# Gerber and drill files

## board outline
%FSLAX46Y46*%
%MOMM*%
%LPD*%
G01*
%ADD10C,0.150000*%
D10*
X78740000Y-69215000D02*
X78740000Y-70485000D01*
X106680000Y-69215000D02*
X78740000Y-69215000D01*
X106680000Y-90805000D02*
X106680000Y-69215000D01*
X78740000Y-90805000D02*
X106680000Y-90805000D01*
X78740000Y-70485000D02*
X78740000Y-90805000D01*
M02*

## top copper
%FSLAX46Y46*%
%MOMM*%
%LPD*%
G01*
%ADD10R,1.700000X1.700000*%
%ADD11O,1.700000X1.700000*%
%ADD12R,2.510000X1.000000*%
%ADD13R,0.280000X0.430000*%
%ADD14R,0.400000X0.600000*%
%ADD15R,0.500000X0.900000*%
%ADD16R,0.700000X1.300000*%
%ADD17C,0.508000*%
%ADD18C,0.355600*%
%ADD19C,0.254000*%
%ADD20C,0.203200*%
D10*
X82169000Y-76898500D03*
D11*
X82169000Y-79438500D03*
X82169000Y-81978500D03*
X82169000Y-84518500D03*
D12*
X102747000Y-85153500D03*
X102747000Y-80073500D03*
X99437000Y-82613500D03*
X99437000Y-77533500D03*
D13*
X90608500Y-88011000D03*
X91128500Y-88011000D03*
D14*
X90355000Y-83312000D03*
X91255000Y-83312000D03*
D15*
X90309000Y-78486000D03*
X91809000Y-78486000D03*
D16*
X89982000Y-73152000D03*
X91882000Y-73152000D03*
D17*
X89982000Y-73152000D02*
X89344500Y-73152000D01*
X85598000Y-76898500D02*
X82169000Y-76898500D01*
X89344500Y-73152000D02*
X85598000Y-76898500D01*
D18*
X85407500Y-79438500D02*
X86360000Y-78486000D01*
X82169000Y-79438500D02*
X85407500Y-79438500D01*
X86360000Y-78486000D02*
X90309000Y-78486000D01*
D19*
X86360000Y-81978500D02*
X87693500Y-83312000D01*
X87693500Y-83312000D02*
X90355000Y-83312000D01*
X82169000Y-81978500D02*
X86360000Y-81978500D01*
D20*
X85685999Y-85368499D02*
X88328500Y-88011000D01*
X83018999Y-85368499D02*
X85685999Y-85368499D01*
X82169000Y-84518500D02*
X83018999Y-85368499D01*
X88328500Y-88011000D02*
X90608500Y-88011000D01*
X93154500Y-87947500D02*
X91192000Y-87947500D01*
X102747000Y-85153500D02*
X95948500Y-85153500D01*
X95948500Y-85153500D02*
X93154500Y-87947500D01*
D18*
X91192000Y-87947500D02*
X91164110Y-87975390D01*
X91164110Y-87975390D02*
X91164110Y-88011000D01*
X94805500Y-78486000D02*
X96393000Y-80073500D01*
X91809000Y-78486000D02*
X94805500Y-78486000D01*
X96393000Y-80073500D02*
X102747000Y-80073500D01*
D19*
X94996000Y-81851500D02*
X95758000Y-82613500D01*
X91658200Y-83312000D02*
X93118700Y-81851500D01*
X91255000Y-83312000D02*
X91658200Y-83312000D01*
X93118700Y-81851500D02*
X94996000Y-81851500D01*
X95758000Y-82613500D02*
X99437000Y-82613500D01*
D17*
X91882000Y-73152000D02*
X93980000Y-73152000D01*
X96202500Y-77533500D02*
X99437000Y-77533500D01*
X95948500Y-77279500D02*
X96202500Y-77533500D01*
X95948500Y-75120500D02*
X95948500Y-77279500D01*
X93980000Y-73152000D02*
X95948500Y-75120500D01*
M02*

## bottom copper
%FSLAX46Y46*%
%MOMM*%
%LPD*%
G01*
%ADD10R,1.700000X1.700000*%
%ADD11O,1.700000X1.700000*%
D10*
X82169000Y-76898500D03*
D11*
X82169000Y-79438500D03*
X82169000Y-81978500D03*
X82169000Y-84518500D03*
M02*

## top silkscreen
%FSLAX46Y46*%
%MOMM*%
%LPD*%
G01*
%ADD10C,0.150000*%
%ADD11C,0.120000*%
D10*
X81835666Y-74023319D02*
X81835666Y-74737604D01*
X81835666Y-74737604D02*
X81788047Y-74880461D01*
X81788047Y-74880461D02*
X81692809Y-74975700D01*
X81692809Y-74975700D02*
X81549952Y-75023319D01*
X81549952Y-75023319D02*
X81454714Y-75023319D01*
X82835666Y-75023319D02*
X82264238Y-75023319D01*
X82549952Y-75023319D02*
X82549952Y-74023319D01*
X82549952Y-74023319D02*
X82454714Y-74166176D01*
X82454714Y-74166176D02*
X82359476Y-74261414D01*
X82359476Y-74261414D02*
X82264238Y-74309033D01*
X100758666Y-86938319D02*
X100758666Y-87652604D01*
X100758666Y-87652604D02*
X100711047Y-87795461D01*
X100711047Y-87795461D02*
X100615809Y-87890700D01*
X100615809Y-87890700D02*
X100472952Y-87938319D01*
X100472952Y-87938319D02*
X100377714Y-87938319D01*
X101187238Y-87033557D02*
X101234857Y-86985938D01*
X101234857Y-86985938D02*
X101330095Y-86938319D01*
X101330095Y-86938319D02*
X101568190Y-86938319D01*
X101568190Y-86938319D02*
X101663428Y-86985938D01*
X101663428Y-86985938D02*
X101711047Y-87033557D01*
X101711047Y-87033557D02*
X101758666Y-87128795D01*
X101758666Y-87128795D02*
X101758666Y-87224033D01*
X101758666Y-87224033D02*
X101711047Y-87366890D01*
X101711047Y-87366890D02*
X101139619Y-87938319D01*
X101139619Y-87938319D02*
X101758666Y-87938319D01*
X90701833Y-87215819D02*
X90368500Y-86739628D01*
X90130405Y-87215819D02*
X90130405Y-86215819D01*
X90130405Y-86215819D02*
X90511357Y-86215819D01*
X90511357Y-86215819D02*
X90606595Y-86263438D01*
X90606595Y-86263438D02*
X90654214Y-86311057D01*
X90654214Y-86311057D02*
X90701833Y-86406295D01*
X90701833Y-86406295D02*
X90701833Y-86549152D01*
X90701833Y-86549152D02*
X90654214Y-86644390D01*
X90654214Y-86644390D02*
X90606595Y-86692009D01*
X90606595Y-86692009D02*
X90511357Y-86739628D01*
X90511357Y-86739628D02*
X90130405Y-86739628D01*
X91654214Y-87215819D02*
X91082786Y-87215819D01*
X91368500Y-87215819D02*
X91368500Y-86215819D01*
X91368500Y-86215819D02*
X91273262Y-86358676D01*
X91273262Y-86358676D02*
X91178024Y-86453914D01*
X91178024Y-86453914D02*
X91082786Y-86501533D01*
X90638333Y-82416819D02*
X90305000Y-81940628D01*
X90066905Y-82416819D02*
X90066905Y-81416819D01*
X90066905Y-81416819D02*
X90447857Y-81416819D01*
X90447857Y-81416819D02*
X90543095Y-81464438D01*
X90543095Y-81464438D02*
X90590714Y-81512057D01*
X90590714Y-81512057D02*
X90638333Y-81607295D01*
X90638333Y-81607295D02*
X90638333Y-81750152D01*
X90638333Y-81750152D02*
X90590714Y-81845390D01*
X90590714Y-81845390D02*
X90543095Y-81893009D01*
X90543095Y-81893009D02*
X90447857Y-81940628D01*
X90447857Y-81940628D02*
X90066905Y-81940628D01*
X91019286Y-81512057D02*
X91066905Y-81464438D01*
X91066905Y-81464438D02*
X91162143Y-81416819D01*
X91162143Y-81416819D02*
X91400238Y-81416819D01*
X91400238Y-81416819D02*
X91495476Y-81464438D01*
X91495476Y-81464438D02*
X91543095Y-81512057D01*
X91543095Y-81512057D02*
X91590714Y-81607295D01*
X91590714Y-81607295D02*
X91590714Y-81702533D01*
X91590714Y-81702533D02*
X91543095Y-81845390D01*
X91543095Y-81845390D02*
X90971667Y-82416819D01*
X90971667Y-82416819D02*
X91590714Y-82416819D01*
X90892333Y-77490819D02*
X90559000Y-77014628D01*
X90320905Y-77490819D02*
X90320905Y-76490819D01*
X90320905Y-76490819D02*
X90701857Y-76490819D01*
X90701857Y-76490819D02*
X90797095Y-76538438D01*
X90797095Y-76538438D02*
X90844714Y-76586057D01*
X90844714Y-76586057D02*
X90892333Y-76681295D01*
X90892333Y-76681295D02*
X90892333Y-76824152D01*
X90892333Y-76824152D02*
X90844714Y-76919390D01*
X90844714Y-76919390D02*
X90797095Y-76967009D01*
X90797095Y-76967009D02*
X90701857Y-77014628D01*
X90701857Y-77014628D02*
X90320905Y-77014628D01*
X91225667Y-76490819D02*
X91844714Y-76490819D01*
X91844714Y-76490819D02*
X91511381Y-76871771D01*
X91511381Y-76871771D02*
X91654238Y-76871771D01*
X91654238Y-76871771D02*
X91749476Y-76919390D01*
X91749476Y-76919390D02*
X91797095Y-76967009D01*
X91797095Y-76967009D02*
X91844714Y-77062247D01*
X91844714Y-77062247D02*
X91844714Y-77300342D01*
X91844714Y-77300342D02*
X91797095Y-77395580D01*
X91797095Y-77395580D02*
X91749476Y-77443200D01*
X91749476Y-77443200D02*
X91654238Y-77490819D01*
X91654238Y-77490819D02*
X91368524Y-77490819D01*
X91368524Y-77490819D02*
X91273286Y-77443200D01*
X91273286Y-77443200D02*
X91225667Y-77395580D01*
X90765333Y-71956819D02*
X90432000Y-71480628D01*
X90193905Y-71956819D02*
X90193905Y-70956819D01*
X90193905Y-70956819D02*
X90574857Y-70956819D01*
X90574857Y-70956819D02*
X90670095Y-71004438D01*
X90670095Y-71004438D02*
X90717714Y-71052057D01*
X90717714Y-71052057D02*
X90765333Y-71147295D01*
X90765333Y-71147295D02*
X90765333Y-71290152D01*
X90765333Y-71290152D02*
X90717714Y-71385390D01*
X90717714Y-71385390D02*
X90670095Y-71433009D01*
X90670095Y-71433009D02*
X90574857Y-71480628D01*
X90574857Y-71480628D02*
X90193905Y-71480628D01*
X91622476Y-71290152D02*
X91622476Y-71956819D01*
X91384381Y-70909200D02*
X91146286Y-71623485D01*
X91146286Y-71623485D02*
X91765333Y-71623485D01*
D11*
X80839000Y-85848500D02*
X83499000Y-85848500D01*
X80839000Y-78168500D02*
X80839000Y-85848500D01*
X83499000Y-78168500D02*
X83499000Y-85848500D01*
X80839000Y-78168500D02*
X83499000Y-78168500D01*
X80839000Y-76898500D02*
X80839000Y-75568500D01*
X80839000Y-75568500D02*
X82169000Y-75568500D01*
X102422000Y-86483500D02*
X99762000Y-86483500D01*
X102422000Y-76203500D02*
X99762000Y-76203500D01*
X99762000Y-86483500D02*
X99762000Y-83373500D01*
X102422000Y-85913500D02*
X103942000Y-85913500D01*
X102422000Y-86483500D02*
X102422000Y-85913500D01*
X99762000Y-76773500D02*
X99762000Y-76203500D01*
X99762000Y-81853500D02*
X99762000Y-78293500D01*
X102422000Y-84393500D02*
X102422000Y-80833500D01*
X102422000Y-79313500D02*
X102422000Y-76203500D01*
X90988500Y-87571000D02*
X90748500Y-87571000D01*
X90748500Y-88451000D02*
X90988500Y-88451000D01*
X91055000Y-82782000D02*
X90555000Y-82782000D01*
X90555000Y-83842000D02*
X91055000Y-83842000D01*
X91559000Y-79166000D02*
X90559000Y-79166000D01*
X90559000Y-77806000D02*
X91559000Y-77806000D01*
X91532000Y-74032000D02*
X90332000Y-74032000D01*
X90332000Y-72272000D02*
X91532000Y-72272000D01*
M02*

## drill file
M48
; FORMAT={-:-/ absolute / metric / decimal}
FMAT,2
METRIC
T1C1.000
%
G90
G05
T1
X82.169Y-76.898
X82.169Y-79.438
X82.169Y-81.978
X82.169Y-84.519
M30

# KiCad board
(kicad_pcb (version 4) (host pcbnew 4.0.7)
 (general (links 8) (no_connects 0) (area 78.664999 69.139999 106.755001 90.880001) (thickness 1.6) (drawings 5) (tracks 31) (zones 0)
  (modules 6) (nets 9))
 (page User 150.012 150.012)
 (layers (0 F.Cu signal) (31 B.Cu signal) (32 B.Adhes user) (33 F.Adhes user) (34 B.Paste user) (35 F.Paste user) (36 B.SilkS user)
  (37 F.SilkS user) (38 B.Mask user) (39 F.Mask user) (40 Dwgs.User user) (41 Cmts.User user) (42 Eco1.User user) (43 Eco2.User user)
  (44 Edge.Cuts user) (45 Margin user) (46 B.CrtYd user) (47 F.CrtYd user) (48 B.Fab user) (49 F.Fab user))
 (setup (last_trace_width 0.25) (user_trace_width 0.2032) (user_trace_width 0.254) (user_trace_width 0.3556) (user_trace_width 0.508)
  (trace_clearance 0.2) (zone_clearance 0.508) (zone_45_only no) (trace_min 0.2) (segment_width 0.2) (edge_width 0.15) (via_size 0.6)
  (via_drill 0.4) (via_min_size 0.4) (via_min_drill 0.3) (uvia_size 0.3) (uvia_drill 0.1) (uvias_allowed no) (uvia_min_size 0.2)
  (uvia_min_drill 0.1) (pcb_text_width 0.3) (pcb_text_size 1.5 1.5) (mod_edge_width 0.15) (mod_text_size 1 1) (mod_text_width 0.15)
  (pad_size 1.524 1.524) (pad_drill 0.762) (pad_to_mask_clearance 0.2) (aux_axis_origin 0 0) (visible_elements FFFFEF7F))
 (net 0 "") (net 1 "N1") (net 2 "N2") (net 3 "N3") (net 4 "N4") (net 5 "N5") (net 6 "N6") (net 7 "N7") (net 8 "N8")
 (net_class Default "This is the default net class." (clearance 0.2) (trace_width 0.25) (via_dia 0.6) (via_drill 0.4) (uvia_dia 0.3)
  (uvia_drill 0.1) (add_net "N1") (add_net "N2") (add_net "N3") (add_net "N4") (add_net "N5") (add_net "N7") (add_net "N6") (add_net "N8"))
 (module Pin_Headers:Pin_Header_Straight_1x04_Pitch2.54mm (layer F.Cu) (at 82.169 76.8985)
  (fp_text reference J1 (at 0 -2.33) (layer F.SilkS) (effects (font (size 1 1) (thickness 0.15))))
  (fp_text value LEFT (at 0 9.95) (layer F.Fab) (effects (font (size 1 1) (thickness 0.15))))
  (fp_line (start -1.33 8.95) (end 1.33 8.95) (layer F.SilkS) (width 0.12))
  (fp_line (start -1.33 1.27) (end -1.33 8.95) (layer F.SilkS) (width 0.12))
  (fp_line (start 1.33 1.27) (end 1.33 8.95) (layer F.SilkS) (width 0.12))
  (fp_line (start -1.33 1.27) (end 1.33 1.27) (layer F.SilkS) (width 0.12))
  (fp_line (start -1.33 0) (end -1.33 -1.33) (layer F.SilkS) (width 0.12))
  (fp_line (start -1.33 -1.33) (end 0 -1.33) (layer F.SilkS) (width 0.12))
  (pad 1 thru_hole rect (at 0 0) (size 1.7 1.7) (drill 1) (layers *.Cu *.Mask) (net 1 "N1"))
  (pad 2 thru_hole oval (at 0 2.54) (size 1.7 1.7) (drill 1) (layers *.Cu *.Mask) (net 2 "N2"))
  (pad 3 thru_hole oval (at 0 5.08) (size 1.7 1.7) (drill 1) (layers *.Cu *.Mask) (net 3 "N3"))
  (pad 4 thru_hole oval (at 0 7.62) (size 1.7 1.7) (drill 1) (layers *.Cu *.Mask) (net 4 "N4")))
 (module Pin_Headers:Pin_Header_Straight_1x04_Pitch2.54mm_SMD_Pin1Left (layer F.Cu) (at 101.092 81.3435 180)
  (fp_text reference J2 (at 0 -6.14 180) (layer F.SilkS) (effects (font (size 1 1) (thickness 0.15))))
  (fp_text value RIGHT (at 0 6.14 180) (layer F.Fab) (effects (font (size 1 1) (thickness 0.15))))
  (fp_line (start -1.33 -5.14) (end 1.33 -5.14) (layer F.SilkS) (width 0.12))
  (fp_line (start -1.33 5.14) (end 1.33 5.14) (layer F.SilkS) (width 0.12))
  (fp_line (start 1.33 -5.14) (end 1.33 -2.03) (layer F.SilkS) (width 0.12))
  (fp_line (start -1.33 -4.57) (end -2.85 -4.57) (layer F.SilkS) (width 0.12))
  (fp_line (start -1.33 -5.14) (end -1.33 -4.57) (layer F.SilkS) (width 0.12))
  (fp_line (start 1.33 4.57) (end 1.33 5.14) (layer F.SilkS) (width 0.12))
  (fp_line (start 1.33 -0.51) (end 1.33 3.05) (layer F.SilkS) (width 0.12))
  (fp_line (start -1.33 -3.05) (end -1.33 0.51) (layer F.SilkS) (width 0.12))
  (fp_line (start -1.33 2.03) (end -1.33 5.14) (layer F.SilkS) (width 0.12))
  (pad 1 smd rect (at -1.655 -3.81 180) (size 2.51 1) (layers F.Cu F.Paste F.Mask) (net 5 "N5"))
  (pad 3 smd rect (at -1.655 1.27 180) (size 2.51 1) (layers F.Cu F.Paste F.Mask) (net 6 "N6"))
  (pad 2 smd rect (at 1.655 -1.27 180) (size 2.51 1) (layers F.Cu F.Paste F.Mask) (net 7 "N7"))
  (pad 4 smd rect (at 1.655 3.81 180) (size 2.51 1) (layers F.Cu F.Paste F.Mask) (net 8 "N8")))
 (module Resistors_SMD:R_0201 (layer F.Cu) (at 90.8685 88.011)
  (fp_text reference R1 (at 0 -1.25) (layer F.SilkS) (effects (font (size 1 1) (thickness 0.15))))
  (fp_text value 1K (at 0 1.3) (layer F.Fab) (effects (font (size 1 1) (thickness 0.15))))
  (fp_line (start 0.12 -0.44) (end -0.12 -0.44) (layer F.SilkS) (width 0.12))
  (fp_line (start -0.12 0.44) (end 0.12 0.44) (layer F.SilkS) (width 0.12))
  (pad 1 smd rect (at -0.26 0) (size 0.28 0.43) (layers F.Cu F.Paste F.Mask) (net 4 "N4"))
  (pad 2 smd rect (at 0.26 0) (size 0.28 0.43) (layers F.Cu F.Paste F.Mask) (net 5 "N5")))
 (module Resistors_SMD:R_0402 (layer F.Cu) (at 90.805 83.312)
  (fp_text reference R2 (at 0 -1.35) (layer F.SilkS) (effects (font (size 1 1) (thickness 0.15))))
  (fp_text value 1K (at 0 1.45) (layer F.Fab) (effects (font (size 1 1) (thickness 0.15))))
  (fp_line (start 0.25 -0.53) (end -0.25 -0.53) (layer F.SilkS) (width 0.12))
  (fp_line (start -0.25 0.53) (end 0.25 0.53) (layer F.SilkS) (width 0.12))
  (pad 1 smd rect (at -0.45 0) (size 0.4 0.6) (layers F.Cu F.Paste F.Mask) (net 3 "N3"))
  (pad 2 smd rect (at 0.45 0) (size 0.4 0.6) (layers F.Cu F.Paste F.Mask) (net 7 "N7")))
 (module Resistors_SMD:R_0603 (layer F.Cu) (at 91.059 78.486)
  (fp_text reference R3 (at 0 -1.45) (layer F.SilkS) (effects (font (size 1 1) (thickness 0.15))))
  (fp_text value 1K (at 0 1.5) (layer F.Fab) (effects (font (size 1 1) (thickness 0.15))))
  (fp_line (start 0.5 0.68) (end -0.5 0.68) (layer F.SilkS) (width 0.12))
  (fp_line (start -0.5 -0.68) (end 0.5 -0.68) (layer F.SilkS) (width 0.12))
  (pad 1 smd rect (at -0.75 0) (size 0.5 0.9) (layers F.Cu F.Paste F.Mask) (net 2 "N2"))
  (pad 2 smd rect (at 0.75 0) (size 0.5 0.9) (layers F.Cu F.Paste F.Mask) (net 6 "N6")))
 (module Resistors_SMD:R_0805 (layer F.Cu) (at 90.932 73.152)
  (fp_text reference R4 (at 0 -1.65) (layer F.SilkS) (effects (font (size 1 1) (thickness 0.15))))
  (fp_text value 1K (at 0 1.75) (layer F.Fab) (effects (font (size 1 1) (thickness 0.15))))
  (fp_line (start 0.6 0.88) (end -0.6 0.88) (layer F.SilkS) (width 0.12))
  (fp_line (start -0.6 -0.88) (end 0.6 -0.88) (layer F.SilkS) (width 0.12))
  (pad 1 smd rect (at -0.95 0) (size 0.7 1.3) (layers F.Cu F.Paste F.Mask) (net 1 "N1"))
  (pad 2 smd rect (at 0.95 0) (size 0.7 1.3) (layers F.Cu F.Paste F.Mask) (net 8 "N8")))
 (gr_line (start 78.74 69.215) (end 78.74 70.485) (layer Edge.Cuts) (width 0.15))
 (gr_line (start 106.68 69.215) (end 78.74 69.215) (layer Edge.Cuts) (width 0.15))
 (gr_line (start 106.68 90.805) (end 106.68 69.215) (layer Edge.Cuts) (width 0.15))
 (gr_line (start 78.74 90.805) (end 106.68 90.805) (layer Edge.Cuts) (width 0.15))
 (gr_line (start 78.74 70.485) (end 78.74 90.805) (layer Edge.Cuts) (width 0.15))
 (segment (start 89.982 73.152) (end 89.3445 73.152) (width 0.508) (layer F.Cu) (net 1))
 (segment (start 85.598 76.8985) (end 82.169 76.8985) (width 0.508) (layer F.Cu) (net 1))
 (segment (start 89.3445 73.152) (end 85.598 76.8985) (width 0.508) (layer F.Cu) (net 1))
 (segment (start 85.4075 79.4385) (end 86.36 78.486) (width 0.3556) (layer F.Cu) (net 2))
 (segment (start 82.169 79.4385) (end 85.4075 79.4385) (width 0.3556) (layer F.Cu) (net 2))
 (segment (start 86.36 78.486) (end 90.309 78.486) (width 0.3556) (layer F.Cu) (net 2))
 (segment (start 86.36 81.9785) (end 87.6935 83.312) (width 0.254) (layer F.Cu) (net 3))
 (segment (start 87.6935 83.312) (end 90.355 83.312) (width 0.254) (layer F.Cu) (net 3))
 (segment (start 82.169 81.9785) (end 86.36 81.9785) (width 0.254) (layer F.Cu) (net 3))
 (segment (start 85.685999 85.368499) (end 88.3285 88.011) (width 0.2032) (layer F.Cu) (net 4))
 (segment (start 83.018999 85.368499) (end 85.685999 85.368499) (width 0.2032) (layer F.Cu) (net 4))
 (segment (start 82.169 84.5185) (end 83.018999 85.368499) (width 0.2032) (layer F.Cu) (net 4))
 (segment (start 88.3285 88.011) (end 90.6085 88.011) (width 0.2032) (layer F.Cu) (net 4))
 (segment (start 93.1545 87.9475) (end 91.192 87.9475) (width 0.2032) (layer F.Cu) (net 5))
 (segment (start 102.747 85.1535) (end 95.9485 85.1535) (width 0.2032) (layer F.Cu) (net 5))
 (segment (start 95.9485 85.1535) (end 93.1545 87.9475) (width 0.2032) (layer F.Cu) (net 5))
 (segment (start 91.192 87.9475) (end 91.16411 87.97539) (width 0.3556) (layer F.Cu) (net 5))
 (segment (start 91.16411 87.97539) (end 91.16411 88.011) (width 0.3556) (layer F.Cu) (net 5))
 (segment (start 94.8055 78.486) (end 96.393 80.0735) (width 0.3556) (layer F.Cu) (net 6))
 (segment (start 91.809 78.486) (end 94.8055 78.486) (width 0.3556) (layer F.Cu) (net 6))
 (segment (start 96.393 80.0735) (end 102.747 80.0735) (width 0.3556) (layer F.Cu) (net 6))
 (segment (start 94.996 81.8515) (end 95.758 82.6135) (width 0.254) (layer F.Cu) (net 7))
 (segment (start 91.6582 83.312) (end 93.1187 81.8515) (width 0.254) (layer F.Cu) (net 7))
 (segment (start 91.255 83.312) (end 91.6582 83.312) (width 0.254) (layer F.Cu) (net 7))
 (segment (start 93.1187 81.8515) (end 94.996 81.8515) (width 0.254) (layer F.Cu) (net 7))
 (segment (start 95.758 82.6135) (end 99.437 82.6135) (width 0.254) (layer F.Cu) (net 7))
 (segment (start 91.882 73.152) (end 93.98 73.152) (width 0.508) (layer F.Cu) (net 8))
 (segment (start 96.2025 77.5335) (end 99.437 77.5335) (width 0.508) (layer F.Cu) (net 8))
 (segment (start 95.9485 77.2795) (end 96.2025 77.5335) (width 0.508) (layer F.Cu) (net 8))
 (segment (start 95.9485 75.1205) (end 95.9485 77.2795) (width 0.508) (layer F.Cu) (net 8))
 (segment (start 93.98 73.152) (end 95.9485 75.1205) (width 0.508) (layer F.Cu) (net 8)))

